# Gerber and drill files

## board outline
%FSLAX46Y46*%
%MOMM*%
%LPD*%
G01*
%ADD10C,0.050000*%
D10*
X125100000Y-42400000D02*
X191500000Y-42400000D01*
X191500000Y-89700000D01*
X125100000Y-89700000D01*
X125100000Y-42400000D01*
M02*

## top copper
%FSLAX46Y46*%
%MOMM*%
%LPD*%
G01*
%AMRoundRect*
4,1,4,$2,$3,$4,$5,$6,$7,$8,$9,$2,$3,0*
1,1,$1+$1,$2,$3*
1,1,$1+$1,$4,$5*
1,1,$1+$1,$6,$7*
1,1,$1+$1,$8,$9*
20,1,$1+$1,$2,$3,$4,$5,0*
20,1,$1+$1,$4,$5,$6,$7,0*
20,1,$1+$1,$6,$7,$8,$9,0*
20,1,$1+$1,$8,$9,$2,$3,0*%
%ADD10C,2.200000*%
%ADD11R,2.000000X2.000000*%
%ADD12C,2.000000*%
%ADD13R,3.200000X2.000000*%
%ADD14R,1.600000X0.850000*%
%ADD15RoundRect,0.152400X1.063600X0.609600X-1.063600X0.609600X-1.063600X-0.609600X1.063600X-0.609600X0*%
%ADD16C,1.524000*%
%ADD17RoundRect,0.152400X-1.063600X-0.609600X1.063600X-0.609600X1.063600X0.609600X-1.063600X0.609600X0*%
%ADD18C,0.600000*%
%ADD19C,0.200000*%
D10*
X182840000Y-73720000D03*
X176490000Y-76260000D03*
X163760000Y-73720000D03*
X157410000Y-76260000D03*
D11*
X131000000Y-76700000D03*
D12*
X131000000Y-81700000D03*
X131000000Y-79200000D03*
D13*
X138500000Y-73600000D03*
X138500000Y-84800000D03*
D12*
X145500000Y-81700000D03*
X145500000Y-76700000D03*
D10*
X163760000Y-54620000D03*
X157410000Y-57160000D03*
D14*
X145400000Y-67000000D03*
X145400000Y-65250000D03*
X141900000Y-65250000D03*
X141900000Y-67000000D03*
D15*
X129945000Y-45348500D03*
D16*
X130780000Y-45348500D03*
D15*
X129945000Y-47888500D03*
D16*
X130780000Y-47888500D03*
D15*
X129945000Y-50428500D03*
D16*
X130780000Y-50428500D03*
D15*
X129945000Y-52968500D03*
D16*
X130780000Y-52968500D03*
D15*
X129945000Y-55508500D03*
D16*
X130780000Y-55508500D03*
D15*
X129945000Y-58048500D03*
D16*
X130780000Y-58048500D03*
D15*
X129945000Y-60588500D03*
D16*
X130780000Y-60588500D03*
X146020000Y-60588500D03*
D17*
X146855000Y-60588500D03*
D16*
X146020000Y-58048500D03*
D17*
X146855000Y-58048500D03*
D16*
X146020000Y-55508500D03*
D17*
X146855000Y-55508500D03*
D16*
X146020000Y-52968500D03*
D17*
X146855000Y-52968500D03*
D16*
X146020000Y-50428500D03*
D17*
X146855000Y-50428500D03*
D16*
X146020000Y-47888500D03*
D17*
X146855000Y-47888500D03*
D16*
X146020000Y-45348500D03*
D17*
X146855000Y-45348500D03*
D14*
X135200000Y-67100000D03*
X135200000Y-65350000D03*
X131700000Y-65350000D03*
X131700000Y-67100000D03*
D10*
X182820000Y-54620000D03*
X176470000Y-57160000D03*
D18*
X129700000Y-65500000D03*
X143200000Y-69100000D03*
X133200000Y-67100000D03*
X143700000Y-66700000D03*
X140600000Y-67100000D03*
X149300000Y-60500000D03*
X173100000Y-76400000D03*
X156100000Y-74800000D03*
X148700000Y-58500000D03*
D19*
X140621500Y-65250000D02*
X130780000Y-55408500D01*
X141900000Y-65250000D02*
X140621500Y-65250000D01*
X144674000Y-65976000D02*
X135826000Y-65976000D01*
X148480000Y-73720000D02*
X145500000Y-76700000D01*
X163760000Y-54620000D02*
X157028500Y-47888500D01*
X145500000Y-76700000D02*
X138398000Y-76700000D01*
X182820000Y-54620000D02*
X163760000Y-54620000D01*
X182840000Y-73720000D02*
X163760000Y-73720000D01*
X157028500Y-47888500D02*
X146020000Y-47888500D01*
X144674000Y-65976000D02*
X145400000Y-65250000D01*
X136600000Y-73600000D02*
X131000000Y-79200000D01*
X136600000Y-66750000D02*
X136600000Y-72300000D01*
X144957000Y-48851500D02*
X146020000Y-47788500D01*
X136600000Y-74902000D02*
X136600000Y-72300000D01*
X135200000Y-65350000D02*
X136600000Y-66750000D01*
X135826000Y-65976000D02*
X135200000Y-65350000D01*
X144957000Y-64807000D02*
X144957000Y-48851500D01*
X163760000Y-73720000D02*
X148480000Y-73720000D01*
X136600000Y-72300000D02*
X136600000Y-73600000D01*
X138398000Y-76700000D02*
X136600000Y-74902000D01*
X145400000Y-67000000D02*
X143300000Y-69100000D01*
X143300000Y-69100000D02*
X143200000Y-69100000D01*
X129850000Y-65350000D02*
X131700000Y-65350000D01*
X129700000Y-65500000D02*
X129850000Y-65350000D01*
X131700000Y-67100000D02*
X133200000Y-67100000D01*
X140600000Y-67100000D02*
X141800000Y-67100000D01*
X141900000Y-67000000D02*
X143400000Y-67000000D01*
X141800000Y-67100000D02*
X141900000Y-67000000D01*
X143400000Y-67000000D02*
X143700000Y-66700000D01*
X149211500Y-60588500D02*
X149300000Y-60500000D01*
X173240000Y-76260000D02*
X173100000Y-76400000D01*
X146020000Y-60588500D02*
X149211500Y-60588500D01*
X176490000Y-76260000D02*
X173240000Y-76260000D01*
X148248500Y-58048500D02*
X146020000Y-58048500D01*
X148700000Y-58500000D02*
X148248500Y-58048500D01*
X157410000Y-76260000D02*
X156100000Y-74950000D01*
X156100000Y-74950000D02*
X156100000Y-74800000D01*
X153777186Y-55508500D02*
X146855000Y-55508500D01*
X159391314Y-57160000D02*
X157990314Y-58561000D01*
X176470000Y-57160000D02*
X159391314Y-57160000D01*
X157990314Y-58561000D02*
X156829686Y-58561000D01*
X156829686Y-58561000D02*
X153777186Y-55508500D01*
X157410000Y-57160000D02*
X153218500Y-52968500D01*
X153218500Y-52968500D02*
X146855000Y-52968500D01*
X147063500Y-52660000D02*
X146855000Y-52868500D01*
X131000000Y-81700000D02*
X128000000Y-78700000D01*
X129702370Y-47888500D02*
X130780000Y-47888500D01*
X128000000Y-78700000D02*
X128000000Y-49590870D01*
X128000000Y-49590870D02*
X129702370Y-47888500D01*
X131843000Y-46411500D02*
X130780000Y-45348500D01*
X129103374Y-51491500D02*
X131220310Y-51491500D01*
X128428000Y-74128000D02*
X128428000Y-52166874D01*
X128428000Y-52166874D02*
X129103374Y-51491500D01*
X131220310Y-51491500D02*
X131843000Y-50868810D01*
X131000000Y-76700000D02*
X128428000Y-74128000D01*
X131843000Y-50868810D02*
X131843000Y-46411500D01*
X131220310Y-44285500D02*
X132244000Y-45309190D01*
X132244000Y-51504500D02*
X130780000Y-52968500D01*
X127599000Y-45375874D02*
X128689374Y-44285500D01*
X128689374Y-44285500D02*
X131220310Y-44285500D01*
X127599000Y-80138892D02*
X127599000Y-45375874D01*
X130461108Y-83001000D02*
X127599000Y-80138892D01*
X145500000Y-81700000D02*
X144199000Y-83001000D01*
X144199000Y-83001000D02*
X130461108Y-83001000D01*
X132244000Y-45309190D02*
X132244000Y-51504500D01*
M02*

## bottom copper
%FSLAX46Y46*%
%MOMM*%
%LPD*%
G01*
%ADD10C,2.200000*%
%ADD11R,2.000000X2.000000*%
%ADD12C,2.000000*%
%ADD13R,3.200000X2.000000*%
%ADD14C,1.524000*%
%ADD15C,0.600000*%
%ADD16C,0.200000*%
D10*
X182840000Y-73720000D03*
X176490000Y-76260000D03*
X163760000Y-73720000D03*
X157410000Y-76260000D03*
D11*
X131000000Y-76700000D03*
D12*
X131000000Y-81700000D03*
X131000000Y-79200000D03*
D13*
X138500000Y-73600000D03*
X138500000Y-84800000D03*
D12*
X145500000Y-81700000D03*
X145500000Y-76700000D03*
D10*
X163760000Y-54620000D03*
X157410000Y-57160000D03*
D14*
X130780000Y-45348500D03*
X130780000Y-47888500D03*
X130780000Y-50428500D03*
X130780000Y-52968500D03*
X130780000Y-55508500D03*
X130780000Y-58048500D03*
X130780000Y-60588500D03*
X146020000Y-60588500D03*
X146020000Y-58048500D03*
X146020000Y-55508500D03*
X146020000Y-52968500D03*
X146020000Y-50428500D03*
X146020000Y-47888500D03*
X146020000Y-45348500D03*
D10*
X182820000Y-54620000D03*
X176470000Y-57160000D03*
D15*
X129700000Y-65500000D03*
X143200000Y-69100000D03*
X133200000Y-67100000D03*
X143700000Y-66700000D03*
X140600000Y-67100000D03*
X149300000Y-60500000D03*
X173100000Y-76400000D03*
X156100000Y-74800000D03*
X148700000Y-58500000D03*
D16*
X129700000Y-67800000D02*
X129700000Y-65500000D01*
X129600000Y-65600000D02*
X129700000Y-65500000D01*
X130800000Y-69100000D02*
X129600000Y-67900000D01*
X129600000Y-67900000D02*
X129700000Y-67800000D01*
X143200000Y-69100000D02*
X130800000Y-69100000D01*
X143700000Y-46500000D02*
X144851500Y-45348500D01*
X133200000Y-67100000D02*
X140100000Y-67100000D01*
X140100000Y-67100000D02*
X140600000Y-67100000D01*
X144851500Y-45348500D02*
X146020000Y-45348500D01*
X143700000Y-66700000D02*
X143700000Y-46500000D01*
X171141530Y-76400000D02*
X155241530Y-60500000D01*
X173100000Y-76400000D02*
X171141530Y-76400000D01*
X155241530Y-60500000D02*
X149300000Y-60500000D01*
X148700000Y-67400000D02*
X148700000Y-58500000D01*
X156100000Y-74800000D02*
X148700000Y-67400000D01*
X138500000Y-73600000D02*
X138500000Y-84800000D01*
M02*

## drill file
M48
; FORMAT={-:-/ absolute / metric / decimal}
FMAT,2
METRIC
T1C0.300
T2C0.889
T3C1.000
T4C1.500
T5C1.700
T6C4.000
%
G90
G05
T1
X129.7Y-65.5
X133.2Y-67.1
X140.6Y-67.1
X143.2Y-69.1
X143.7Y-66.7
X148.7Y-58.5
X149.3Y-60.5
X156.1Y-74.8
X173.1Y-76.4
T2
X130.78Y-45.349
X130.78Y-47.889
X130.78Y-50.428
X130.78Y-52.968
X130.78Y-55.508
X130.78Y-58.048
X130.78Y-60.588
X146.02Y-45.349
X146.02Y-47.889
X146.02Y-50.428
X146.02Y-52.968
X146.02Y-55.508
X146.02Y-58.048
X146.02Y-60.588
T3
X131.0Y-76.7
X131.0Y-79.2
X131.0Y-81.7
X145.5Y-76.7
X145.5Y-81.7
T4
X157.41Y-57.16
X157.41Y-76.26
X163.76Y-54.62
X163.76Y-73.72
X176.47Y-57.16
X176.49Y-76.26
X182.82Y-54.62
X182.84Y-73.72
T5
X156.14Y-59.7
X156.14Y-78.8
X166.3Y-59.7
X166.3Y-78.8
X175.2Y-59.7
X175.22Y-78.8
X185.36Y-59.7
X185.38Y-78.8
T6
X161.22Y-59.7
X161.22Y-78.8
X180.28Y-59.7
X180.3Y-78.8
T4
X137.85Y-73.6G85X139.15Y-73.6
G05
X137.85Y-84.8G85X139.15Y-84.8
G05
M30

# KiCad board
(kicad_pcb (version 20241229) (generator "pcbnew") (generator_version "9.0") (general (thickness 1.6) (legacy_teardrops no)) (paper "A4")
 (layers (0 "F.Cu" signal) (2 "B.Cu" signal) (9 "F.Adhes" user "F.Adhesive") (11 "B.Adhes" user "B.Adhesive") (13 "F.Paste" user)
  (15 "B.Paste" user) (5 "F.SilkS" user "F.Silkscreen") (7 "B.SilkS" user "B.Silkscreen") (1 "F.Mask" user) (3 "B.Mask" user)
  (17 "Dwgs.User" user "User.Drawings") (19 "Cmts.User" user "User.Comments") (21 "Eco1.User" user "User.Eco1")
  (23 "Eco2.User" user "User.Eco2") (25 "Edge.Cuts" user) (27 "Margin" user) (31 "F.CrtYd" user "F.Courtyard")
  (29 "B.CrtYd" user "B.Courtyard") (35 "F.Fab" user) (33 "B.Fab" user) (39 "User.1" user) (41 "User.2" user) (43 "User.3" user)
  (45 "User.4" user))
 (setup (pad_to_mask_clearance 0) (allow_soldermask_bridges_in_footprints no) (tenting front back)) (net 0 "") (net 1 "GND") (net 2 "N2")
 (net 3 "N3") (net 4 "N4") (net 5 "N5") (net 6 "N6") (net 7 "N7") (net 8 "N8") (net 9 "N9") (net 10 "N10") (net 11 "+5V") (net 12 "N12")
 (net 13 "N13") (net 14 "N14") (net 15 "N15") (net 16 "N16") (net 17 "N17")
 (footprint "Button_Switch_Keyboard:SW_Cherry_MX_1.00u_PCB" (layer "F.Cu") (at 182.84 73.72)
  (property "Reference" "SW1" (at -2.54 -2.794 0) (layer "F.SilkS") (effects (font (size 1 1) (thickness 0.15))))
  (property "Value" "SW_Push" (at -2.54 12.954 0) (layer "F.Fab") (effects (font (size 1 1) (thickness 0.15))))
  (pad "" np_thru_hole circle (at -7.62 5.08) (size 1.7 1.7) (drill 1.7) (layers "*.Cu" "*.Mask"))
  (pad "" np_thru_hole circle (at -2.54 5.08) (size 4 4) (drill 4) (layers "*.Cu" "*.Mask"))
  (pad "" np_thru_hole circle (at 2.54 5.08) (size 1.7 1.7) (drill 1.7) (layers "*.Cu" "*.Mask"))
  (pad "1" thru_hole circle (at 0 0) (size 2.2 2.2) (drill 1.5) (layers "*.Cu" "*.Mask") (remove_unused_layers no) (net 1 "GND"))
  (pad "2" thru_hole circle (at -6.35 2.54) (size 2.2 2.2) (drill 1.5) (layers "*.Cu" "*.Mask") (remove_unused_layers no) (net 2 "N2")))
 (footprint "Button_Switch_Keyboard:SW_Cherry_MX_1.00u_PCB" (layer "F.Cu") (at 163.76 73.72)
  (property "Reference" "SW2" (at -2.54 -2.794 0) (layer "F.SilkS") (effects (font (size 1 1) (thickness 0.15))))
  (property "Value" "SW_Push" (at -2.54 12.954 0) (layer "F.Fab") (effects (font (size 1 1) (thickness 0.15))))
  (pad "" np_thru_hole circle (at -7.62 5.08) (size 1.7 1.7) (drill 1.7) (layers "*.Cu" "*.Mask"))
  (pad "" np_thru_hole circle (at -2.54 5.08) (size 4 4) (drill 4) (layers "*.Cu" "*.Mask"))
  (pad "" np_thru_hole circle (at 2.54 5.08) (size 1.7 1.7) (drill 1.7) (layers "*.Cu" "*.Mask"))
  (pad "1" thru_hole circle (at 0 0) (size 2.2 2.2) (drill 1.5) (layers "*.Cu" "*.Mask") (remove_unused_layers no) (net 1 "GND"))
  (pad "2" thru_hole circle (at -6.35 2.54) (size 2.2 2.2) (drill 1.5) (layers "*.Cu" "*.Mask") (remove_unused_layers no) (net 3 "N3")))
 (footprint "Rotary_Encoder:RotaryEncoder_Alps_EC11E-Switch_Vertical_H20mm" (layer "F.Cu") (at 131 76.7)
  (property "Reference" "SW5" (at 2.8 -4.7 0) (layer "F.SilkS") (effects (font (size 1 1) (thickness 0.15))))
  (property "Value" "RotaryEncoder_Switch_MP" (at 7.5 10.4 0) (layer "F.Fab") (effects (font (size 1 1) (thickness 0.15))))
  (pad "A" thru_hole rect (at 0 0) (size 2 2) (drill 1) (layers "*.Cu" "*.Mask") (remove_unused_layers no) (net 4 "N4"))
  (pad "B" thru_hole circle (at 0 5) (size 2 2) (drill 1) (layers "*.Cu" "*.Mask") (remove_unused_layers no) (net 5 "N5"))
  (pad "C" thru_hole circle (at 0 2.5) (size 2 2) (drill 1) (layers "*.Cu" "*.Mask") (remove_unused_layers no) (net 1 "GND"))
  (pad "MP" thru_hole rect (at 7.5 -3.1) (size 3.2 2) (drill oval 2.8 1.5) (layers "*.Cu" "*.Mask") (remove_unused_layers no) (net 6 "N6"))
  (pad "MP" thru_hole rect (at 7.5 8.1) (size 3.2 2) (drill oval 2.8 1.5) (layers "*.Cu" "*.Mask") (remove_unused_layers no) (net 6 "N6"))
  (pad "S1" thru_hole circle (at 14.5 5) (size 2 2) (drill 1) (layers "*.Cu" "*.Mask") (remove_unused_layers no) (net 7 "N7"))
  (pad "S2" thru_hole circle (at 14.5 0) (size 2 2) (drill 1) (layers "*.Cu" "*.Mask") (remove_unused_layers no) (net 1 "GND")))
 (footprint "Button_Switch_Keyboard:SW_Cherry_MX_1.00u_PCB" (layer "F.Cu") (at 163.76 54.62)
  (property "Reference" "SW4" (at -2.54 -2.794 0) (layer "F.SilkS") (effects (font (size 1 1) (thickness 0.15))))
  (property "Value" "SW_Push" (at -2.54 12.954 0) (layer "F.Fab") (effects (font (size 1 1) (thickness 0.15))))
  (pad "" np_thru_hole circle (at -7.62 5.08) (size 1.7 1.7) (drill 1.7) (layers "*.Cu" "*.Mask"))
  (pad "" np_thru_hole circle (at -2.54 5.08) (size 4 4) (drill 4) (layers "*.Cu" "*.Mask"))
  (pad "" np_thru_hole circle (at 2.54 5.08) (size 1.7 1.7) (drill 1.7) (layers "*.Cu" "*.Mask"))
  (pad "1" thru_hole circle (at 0 0) (size 2.2 2.2) (drill 1.5) (layers "*.Cu" "*.Mask") (remove_unused_layers no) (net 1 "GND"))
  (pad "2" thru_hole circle (at -6.35 2.54) (size 2.2 2.2) (drill 1.5) (layers "*.Cu" "*.Mask") (remove_unused_layers no) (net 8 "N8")))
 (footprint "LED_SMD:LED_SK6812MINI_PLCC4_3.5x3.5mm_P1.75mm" (layer "F.Cu") (at 143.65 66.125 180)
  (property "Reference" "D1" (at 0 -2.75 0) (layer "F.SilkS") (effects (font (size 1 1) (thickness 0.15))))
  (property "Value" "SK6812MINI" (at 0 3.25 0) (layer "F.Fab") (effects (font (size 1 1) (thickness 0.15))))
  (pad "1" smd rect (at -1.75 -0.875 180) (size 1.6 0.85) (layers "F.Cu" "F.Mask" "F.Paste") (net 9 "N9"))
  (pad "2" smd rect (at -1.75 0.875 180) (size 1.6 0.85) (layers "F.Cu" "F.Mask" "F.Paste") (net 1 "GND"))
  (pad "3" smd rect (at 1.75 0.875 180) (size 1.6 0.85) (layers "F.Cu" "F.Mask" "F.Paste") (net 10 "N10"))
  (pad "4" smd rect (at 1.75 -0.875 180) (size 1.6 0.85) (layers "F.Cu" "F.Mask" "F.Paste") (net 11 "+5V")))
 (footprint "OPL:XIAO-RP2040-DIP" (layer "F.Cu") (at 138.4 52.9685)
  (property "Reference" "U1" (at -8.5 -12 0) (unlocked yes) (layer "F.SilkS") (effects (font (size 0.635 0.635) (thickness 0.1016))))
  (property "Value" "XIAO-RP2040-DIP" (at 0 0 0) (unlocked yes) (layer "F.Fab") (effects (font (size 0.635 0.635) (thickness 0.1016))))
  (pad "1" smd roundrect (at -8.455 -7.62 180) (size 2.432 1.524) (layers "F.Cu" "F.Mask") (roundrect_rratio 0.1) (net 4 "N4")
   (thermal_bridge_angle 45))
  (pad "1" thru_hole circle (at -7.62 -7.62 180) (size 1.524 1.524) (drill 0.889) (layers "*.Cu" "*.Mask") (remove_unused_layers no)
   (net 4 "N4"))
  (pad "2" smd roundrect (at -8.455 -5.08 180) (size 2.432 1.524) (layers "F.Cu" "F.Mask") (roundrect_rratio 0.1) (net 5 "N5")
   (thermal_bridge_angle 45))
  (pad "2" thru_hole circle (at -7.62 -5.08 180) (size 1.524 1.524) (drill 0.889) (layers "*.Cu" "*.Mask") (remove_unused_layers no)
   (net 5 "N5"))
  (pad "3" smd roundrect (at -8.455 -2.54 180) (size 2.432 1.524) (layers "F.Cu" "F.Mask") (roundrect_rratio 0.1) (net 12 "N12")
   (thermal_bridge_angle 45))
  (pad "3" thru_hole circle (at -7.62 -2.54 180) (size 1.524 1.524) (drill 0.889) (layers "*.Cu" "*.Mask") (remove_unused_layers no)
   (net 12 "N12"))
  (pad "4" smd roundrect (at -8.455 0 180) (size 2.432 1.524) (layers "F.Cu" "F.Mask") (roundrect_rratio 0.1) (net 7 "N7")
   (thermal_bridge_angle 45))
  (pad "4" thru_hole circle (at -7.62 0 180) (size 1.524 1.524) (drill 0.889) (layers "*.Cu" "*.Mask") (remove_unused_layers no)
   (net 7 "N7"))
  (pad "5" smd roundrect (at -8.455 2.54 180) (size 2.432 1.524) (layers "F.Cu" "F.Mask") (roundrect_rratio 0.1) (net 10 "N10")
   (thermal_bridge_angle 45))
  (pad "5" thru_hole circle (at -7.62 2.54 180) (size 1.524 1.524) (drill 0.889) (layers "*.Cu" "*.Mask") (remove_unused_layers no)
   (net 10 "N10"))
  (pad "6" smd roundrect (at -8.455 5.08 180) (size 2.432 1.524) (layers "F.Cu" "F.Mask") (roundrect_rratio 0.1) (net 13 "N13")
   (thermal_bridge_angle 45))
  (pad "6" thru_hole circle (at -7.62 5.08 180) (size 1.524 1.524) (drill 0.889) (layers "*.Cu" "*.Mask") (remove_unused_layers no)
   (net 13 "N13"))
  (pad "7" smd roundrect (at -8.455 7.62 180) (size 2.432 1.524) (layers "F.Cu" "F.Mask") (roundrect_rratio 0.1) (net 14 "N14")
   (thermal_bridge_angle 45))
  (pad "7" thru_hole circle (at -7.62 7.62 180) (size 1.524 1.524) (drill 0.889) (layers "*.Cu" "*.Mask") (remove_unused_layers no)
   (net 14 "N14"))
  (pad "8" thru_hole circle (at 7.62 7.62) (size 1.524 1.524) (drill 0.889) (layers "*.Cu" "*.Mask") (remove_unused_layers no) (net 2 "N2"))
  (pad "8" smd roundrect (at 8.455 7.62) (size 2.432 1.524) (layers "F.Cu" "F.Mask") (roundrect_rratio 0.1) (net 2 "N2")
   (thermal_bridge_angle 45))
  (pad "9" thru_hole circle (at 7.62 5.08) (size 1.524 1.524) (drill 0.889) (layers "*.Cu" "*.Mask") (remove_unused_layers no) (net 3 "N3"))
  (pad "9" smd roundrect (at 8.455 5.08) (size 2.432 1.524) (layers "F.Cu" "F.Mask") (roundrect_rratio 0.1) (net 3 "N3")
   (thermal_bridge_angle 45))
  (pad "10" thru_hole circle (at 7.62 2.54) (size 1.524 1.524) (drill 0.889) (layers "*.Cu" "*.Mask") (remove_unused_layers no)
   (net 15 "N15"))
  (pad "10" smd roundrect (at 8.455 2.54) (size 2.432 1.524) (layers "F.Cu" "F.Mask") (roundrect_rratio 0.1) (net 15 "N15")
   (thermal_bridge_angle 45))
  (pad "11" thru_hole circle (at 7.62 0) (size 1.524 1.524) (drill 0.889) (layers "*.Cu" "*.Mask") (remove_unused_layers no) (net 8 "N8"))
  (pad "11" smd roundrect (at 8.455 0) (size 2.432 1.524) (layers "F.Cu" "F.Mask") (roundrect_rratio 0.1) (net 8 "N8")
   (thermal_bridge_angle 45))
  (pad "12" thru_hole circle (at 7.62 -2.54) (size 1.524 1.524) (drill 0.889) (layers "*.Cu" "*.Mask") (remove_unused_layers no)
   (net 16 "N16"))
  (pad "12" smd roundrect (at 8.455 -2.54) (size 2.432 1.524) (layers "F.Cu" "F.Mask") (roundrect_rratio 0.1) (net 16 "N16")
   (thermal_bridge_angle 45))
  (pad "13" thru_hole circle (at 7.62 -5.08) (size 1.524 1.524) (drill 0.889) (layers "*.Cu" "*.Mask") (remove_unused_layers no)
   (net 1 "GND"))
  (pad "13" smd roundrect (at 8.455 -5.08) (size 2.432 1.524) (layers "F.Cu" "F.Mask") (roundrect_rratio 0.1) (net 1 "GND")
   (thermal_bridge_angle 45))
  (pad "14" thru_hole circle (at 7.62 -7.62) (size 1.524 1.524) (drill 0.889) (layers "*.Cu" "*.Mask") (remove_unused_layers no)
   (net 11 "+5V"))
  (pad "14" smd roundrect (at 8.455 -7.62) (size 2.432 1.524) (layers "F.Cu" "F.Mask") (roundrect_rratio 0.1) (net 11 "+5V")
   (thermal_bridge_angle 45)))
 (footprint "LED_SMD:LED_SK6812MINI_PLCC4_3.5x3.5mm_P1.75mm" (layer "F.Cu") (at 133.45 66.225 180)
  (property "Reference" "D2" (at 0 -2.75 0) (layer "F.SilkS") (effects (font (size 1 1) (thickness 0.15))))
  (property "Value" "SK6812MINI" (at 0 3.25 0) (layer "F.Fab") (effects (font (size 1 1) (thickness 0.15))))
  (pad "1" smd rect (at -1.75 -0.875 180) (size 1.6 0.85) (layers "F.Cu" "F.Mask" "F.Paste") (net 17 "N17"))
  (pad "2" smd rect (at -1.75 0.875 180) (size 1.6 0.85) (layers "F.Cu" "F.Mask" "F.Paste") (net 1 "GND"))
  (pad "3" smd rect (at 1.75 0.875 180) (size 1.6 0.85) (layers "F.Cu" "F.Mask" "F.Paste") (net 9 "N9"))
  (pad "4" smd rect (at 1.75 -0.875 180) (size 1.6 0.85) (layers "F.Cu" "F.Mask" "F.Paste") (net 11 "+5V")))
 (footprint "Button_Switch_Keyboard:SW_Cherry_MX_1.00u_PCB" (layer "F.Cu") (at 182.82 54.62)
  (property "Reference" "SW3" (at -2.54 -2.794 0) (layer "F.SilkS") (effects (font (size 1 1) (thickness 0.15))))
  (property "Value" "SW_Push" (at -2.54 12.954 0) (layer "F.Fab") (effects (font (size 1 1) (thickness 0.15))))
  (pad "" np_thru_hole circle (at -7.62 5.08) (size 1.7 1.7) (drill 1.7) (layers "*.Cu" "*.Mask"))
  (pad "" np_thru_hole circle (at -2.54 5.08) (size 4 4) (drill 4) (layers "*.Cu" "*.Mask"))
  (pad "" np_thru_hole circle (at 2.54 5.08) (size 1.7 1.7) (drill 1.7) (layers "*.Cu" "*.Mask"))
  (pad "1" thru_hole circle (at 0 0) (size 2.2 2.2) (drill 1.5) (layers "*.Cu" "*.Mask") (remove_unused_layers no) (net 1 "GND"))
  (pad "2" thru_hole circle (at -6.35 2.54) (size 2.2 2.2) (drill 1.5) (layers "*.Cu" "*.Mask") (remove_unused_layers no) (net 15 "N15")))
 (gr_rect (start 125.1 42.4) (end 191.5 89.7) (stroke (width 0.05) (type default)) (fill no) (layer "Edge.Cuts"))
 (segment (start 140.6215 65.25) (end 130.78 55.4085) (width 0.2) (layer "F.Cu") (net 10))
 (segment (start 141.9 65.25) (end 140.6215 65.25) (width 0.2) (layer "F.Cu") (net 10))
 (segment (start 144.674 65.976) (end 135.826 65.976) (width 0.2) (layer "F.Cu") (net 1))
 (segment (start 148.48 73.72) (end 145.5 76.7) (width 0.2) (layer "F.Cu") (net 1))
 (segment (start 163.76 54.62) (end 157.0285 47.8885) (width 0.2) (layer "F.Cu") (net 1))
 (segment (start 145.5 76.7) (end 138.398 76.7) (width 0.2) (layer "F.Cu") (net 1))
 (segment (start 182.82 54.62) (end 163.76 54.62) (width 0.2) (layer "F.Cu") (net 1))
 (segment (start 182.84 73.72) (end 163.76 73.72) (width 0.2) (layer "F.Cu") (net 1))
 (segment (start 157.0285 47.8885) (end 146.02 47.8885) (width 0.2) (layer "F.Cu") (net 1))
 (segment (start 144.674 65.976) (end 145.4 65.25) (width 0.2) (layer "F.Cu") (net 1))
 (segment (start 136.6 73.6) (end 131 79.2) (width 0.2) (layer "F.Cu") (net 1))
 (segment (start 136.6 66.75) (end 136.6 72.3) (width 0.2) (layer "F.Cu") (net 1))
 (segment (start 144.957 48.8515) (end 146.02 47.7885) (width 0.2) (layer "F.Cu") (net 1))
 (segment (start 136.6 74.902) (end 136.6 72.3) (width 0.2) (layer "F.Cu") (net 1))
 (segment (start 135.2 65.35) (end 136.6 66.75) (width 0.2) (layer "F.Cu") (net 1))
 (segment (start 135.826 65.976) (end 135.2 65.35) (width 0.2) (layer "F.Cu") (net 1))
 (segment (start 144.957 64.807) (end 144.957 48.8515) (width 0.2) (layer "F.Cu") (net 1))
 (segment (start 163.76 73.72) (end 148.48 73.72) (width 0.2) (layer "F.Cu") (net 1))
 (segment (start 136.6 72.3) (end 136.6 73.6) (width 0.2) (layer "F.Cu") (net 1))
 (segment (start 138.398 76.7) (end 136.6 74.902) (width 0.2) (layer "F.Cu") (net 1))
 (segment (start 145.4 67) (end 143.3 69.1) (width 0.2) (layer "F.Cu") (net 9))
 (segment (start 143.3 69.1) (end 143.2 69.1) (width 0.2) (layer "F.Cu") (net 9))
 (segment (start 129.85 65.35) (end 131.7 65.35) (width 0.2) (layer "F.Cu") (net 9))
 (segment (start 129.7 65.5) (end 129.85 65.35) (width 0.2) (layer "F.Cu") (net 9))
 (via (at 129.7 65.5) (size 0.6) (drill 0.3) (layers "F.Cu" "B.Cu") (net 9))
 (via (at 143.2 69.1) (size 0.6) (drill 0.3) (layers "F.Cu" "B.Cu") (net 9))
 (segment (start 129.7 67.8) (end 129.7 65.5) (width 0.2) (layer "B.Cu") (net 9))
 (segment (start 129.6 65.6) (end 129.7 65.5) (width 0.2) (layer "B.Cu") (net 9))
 (segment (start 130.8 69.1) (end 129.6 67.9) (width 0.2) (layer "B.Cu") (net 9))
 (segment (start 129.6 67.9) (end 129.7 67.8) (width 0.2) (layer "B.Cu") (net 9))
 (segment (start 143.2 69.1) (end 130.8 69.1) (width 0.2) (layer "B.Cu") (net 9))
 (segment (start 131.7 67.1) (end 133.2 67.1) (width 0.2) (layer "F.Cu") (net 11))
 (segment (start 140.6 67.1) (end 141.8 67.1) (width 0.2) (layer "F.Cu") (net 11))
 (segment (start 141.9 67) (end 143.4 67) (width 0.2) (layer "F.Cu") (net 11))
 (segment (start 141.8 67.1) (end 141.9 67) (width 0.2) (layer "F.Cu") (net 11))
 (segment (start 143.4 67) (end 143.7 66.7) (width 0.2) (layer "F.Cu") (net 11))
 (via (at 133.2 67.1) (size 0.6) (drill 0.3) (layers "F.Cu" "B.Cu") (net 11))
 (via (at 143.7 66.7) (size 0.6) (drill 0.3) (layers "F.Cu" "B.Cu") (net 11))
 (via (at 140.6 67.1) (size 0.6) (drill 0.3) (layers "F.Cu" "B.Cu") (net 11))
 (segment (start 143.7 46.5) (end 144.8515 45.3485) (width 0.2) (layer "B.Cu") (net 11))
 (segment (start 133.2 67.1) (end 140.1 67.1) (width 0.2) (layer "B.Cu") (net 11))
 (segment (start 140.1 67.1) (end 140.6 67.1) (width 0.2) (layer "B.Cu") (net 11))
 (segment (start 144.8515 45.3485) (end 146.02 45.3485) (width 0.2) (layer "B.Cu") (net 11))
 (segment (start 143.7 66.7) (end 143.7 46.5) (width 0.2) (layer "B.Cu") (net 11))
 (segment (start 149.2115 60.5885) (end 149.3 60.5) (width 0.2) (layer "F.Cu") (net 2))
 (segment (start 173.24 76.26) (end 173.1 76.4) (width 0.2) (layer "F.Cu") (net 2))
 (segment (start 146.02 60.5885) (end 149.2115 60.5885) (width 0.2) (layer "F.Cu") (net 2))
 (segment (start 176.49 76.26) (end 173.24 76.26) (width 0.2) (layer "F.Cu") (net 2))
 (via (at 149.3 60.5) (size 0.6) (drill 0.3) (layers "F.Cu" "B.Cu") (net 2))
 (via (at 173.1 76.4) (size 0.6) (drill 0.3) (layers "F.Cu" "B.Cu") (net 2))
 (segment (start 171.14153 76.4) (end 155.24153 60.5) (width 0.2) (layer "B.Cu") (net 2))
 (segment (start 173.1 76.4) (end 171.14153 76.4) (width 0.2) (layer "B.Cu") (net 2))
 (segment (start 155.24153 60.5) (end 149.3 60.5) (width 0.2) (layer "B.Cu") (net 2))
 (segment (start 148.2485 58.0485) (end 146.02 58.0485) (width 0.2) (layer "F.Cu") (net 3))
 (segment (start 148.7 58.5) (end 148.2485 58.0485) (width 0.2) (layer "F.Cu") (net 3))
 (segment (start 157.41 76.26) (end 156.1 74.95) (width 0.2) (layer "F.Cu") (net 3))
 (segment (start 156.1 74.95) (end 156.1 74.8) (width 0.2) (layer "F.Cu") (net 3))
 (via (at 156.1 74.8) (size 0.6) (drill 0.3) (layers "F.Cu" "B.Cu") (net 3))
 (via (at 148.7 58.5) (size 0.6) (drill 0.3) (layers "F.Cu" "B.Cu") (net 3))
 (segment (start 148.7 67.4) (end 148.7 58.5) (width 0.2) (layer "B.Cu") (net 3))
 (segment (start 156.1 74.8) (end 148.7 67.4) (width 0.2) (layer "B.Cu") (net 3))
 (segment (start 153.777186 55.5085) (end 146.855 55.5085) (width 0.2) (layer "F.Cu") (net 15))
 (segment (start 159.391314 57.16) (end 157.990314 58.561) (width 0.2) (layer "F.Cu") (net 15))
 (segment (start 176.47 57.16) (end 159.391314 57.16) (width 0.2) (layer "F.Cu") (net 15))
 (segment (start 157.990314 58.561) (end 156.829686 58.561) (width 0.2) (layer "F.Cu") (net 15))
 (segment (start 156.829686 58.561) (end 153.777186 55.5085) (width 0.2) (layer "F.Cu") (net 15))
 (segment (start 157.41 57.16) (end 153.2185 52.9685) (width 0.2) (layer "F.Cu") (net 8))
 (segment (start 153.2185 52.9685) (end 146.855 52.9685) (width 0.2) (layer "F.Cu") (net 8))
 (segment (start 147.0635 52.66) (end 146.855 52.8685) (width 0.2) (layer "F.Cu") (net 8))
 (segment (start 131 81.7) (end 128 78.7) (width 0.2) (layer "F.Cu") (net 5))
 (segment (start 129.70237 47.8885) (end 130.78 47.8885) (width 0.2) (layer "F.Cu") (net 5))
 (segment (start 128 78.7) (end 128 49.59087) (width 0.2) (layer "F.Cu") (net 5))
 (segment (start 128 49.59087) (end 129.70237 47.8885) (width 0.2) (layer "F.Cu") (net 5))
 (segment (start 131.843 46.4115) (end 130.78 45.3485) (width 0.2) (layer "F.Cu") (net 4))
 (segment (start 129.103374 51.4915) (end 131.22031 51.4915) (width 0.2) (layer "F.Cu") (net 4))
 (segment (start 128.428 74.128) (end 128.428 52.166874) (width 0.2) (layer "F.Cu") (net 4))
 (segment (start 128.428 52.166874) (end 129.103374 51.4915) (width 0.2) (layer "F.Cu") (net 4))
 (segment (start 131.22031 51.4915) (end 131.843 50.86881) (width 0.2) (layer "F.Cu") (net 4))
 (segment (start 131 76.7) (end 128.428 74.128) (width 0.2) (layer "F.Cu") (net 4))
 (segment (start 131.843 50.86881) (end 131.843 46.4115) (width 0.2) (layer "F.Cu") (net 4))
 (segment (start 131.22031 44.2855) (end 132.244 45.30919) (width 0.2) (layer "F.Cu") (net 7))
 (segment (start 132.244 51.5045) (end 130.78 52.9685) (width 0.2) (layer "F.Cu") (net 7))
 (segment (start 127.599 45.375874) (end 128.689374 44.2855) (width 0.2) (layer "F.Cu") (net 7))
 (segment (start 128.689374 44.2855) (end 131.22031 44.2855) (width 0.2) (layer "F.Cu") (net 7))
 (segment (start 127.599 80.138892) (end 127.599 45.375874) (width 0.2) (layer "F.Cu") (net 7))
 (segment (start 130.461108 83.001) (end 127.599 80.138892) (width 0.2) (layer "F.Cu") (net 7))
 (segment (start 145.5 81.7) (end 144.199 83.001) (width 0.2) (layer "F.Cu") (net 7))
 (segment (start 144.199 83.001) (end 130.461108 83.001) (width 0.2) (layer "F.Cu") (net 7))
 (segment (start 132.244 45.30919) (end 132.244 51.5045) (width 0.2) (layer "F.Cu") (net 7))
 (segment (start 138.5 73.6) (end 138.5 84.8) (width 0.2) (layer "B.Cu") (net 6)))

